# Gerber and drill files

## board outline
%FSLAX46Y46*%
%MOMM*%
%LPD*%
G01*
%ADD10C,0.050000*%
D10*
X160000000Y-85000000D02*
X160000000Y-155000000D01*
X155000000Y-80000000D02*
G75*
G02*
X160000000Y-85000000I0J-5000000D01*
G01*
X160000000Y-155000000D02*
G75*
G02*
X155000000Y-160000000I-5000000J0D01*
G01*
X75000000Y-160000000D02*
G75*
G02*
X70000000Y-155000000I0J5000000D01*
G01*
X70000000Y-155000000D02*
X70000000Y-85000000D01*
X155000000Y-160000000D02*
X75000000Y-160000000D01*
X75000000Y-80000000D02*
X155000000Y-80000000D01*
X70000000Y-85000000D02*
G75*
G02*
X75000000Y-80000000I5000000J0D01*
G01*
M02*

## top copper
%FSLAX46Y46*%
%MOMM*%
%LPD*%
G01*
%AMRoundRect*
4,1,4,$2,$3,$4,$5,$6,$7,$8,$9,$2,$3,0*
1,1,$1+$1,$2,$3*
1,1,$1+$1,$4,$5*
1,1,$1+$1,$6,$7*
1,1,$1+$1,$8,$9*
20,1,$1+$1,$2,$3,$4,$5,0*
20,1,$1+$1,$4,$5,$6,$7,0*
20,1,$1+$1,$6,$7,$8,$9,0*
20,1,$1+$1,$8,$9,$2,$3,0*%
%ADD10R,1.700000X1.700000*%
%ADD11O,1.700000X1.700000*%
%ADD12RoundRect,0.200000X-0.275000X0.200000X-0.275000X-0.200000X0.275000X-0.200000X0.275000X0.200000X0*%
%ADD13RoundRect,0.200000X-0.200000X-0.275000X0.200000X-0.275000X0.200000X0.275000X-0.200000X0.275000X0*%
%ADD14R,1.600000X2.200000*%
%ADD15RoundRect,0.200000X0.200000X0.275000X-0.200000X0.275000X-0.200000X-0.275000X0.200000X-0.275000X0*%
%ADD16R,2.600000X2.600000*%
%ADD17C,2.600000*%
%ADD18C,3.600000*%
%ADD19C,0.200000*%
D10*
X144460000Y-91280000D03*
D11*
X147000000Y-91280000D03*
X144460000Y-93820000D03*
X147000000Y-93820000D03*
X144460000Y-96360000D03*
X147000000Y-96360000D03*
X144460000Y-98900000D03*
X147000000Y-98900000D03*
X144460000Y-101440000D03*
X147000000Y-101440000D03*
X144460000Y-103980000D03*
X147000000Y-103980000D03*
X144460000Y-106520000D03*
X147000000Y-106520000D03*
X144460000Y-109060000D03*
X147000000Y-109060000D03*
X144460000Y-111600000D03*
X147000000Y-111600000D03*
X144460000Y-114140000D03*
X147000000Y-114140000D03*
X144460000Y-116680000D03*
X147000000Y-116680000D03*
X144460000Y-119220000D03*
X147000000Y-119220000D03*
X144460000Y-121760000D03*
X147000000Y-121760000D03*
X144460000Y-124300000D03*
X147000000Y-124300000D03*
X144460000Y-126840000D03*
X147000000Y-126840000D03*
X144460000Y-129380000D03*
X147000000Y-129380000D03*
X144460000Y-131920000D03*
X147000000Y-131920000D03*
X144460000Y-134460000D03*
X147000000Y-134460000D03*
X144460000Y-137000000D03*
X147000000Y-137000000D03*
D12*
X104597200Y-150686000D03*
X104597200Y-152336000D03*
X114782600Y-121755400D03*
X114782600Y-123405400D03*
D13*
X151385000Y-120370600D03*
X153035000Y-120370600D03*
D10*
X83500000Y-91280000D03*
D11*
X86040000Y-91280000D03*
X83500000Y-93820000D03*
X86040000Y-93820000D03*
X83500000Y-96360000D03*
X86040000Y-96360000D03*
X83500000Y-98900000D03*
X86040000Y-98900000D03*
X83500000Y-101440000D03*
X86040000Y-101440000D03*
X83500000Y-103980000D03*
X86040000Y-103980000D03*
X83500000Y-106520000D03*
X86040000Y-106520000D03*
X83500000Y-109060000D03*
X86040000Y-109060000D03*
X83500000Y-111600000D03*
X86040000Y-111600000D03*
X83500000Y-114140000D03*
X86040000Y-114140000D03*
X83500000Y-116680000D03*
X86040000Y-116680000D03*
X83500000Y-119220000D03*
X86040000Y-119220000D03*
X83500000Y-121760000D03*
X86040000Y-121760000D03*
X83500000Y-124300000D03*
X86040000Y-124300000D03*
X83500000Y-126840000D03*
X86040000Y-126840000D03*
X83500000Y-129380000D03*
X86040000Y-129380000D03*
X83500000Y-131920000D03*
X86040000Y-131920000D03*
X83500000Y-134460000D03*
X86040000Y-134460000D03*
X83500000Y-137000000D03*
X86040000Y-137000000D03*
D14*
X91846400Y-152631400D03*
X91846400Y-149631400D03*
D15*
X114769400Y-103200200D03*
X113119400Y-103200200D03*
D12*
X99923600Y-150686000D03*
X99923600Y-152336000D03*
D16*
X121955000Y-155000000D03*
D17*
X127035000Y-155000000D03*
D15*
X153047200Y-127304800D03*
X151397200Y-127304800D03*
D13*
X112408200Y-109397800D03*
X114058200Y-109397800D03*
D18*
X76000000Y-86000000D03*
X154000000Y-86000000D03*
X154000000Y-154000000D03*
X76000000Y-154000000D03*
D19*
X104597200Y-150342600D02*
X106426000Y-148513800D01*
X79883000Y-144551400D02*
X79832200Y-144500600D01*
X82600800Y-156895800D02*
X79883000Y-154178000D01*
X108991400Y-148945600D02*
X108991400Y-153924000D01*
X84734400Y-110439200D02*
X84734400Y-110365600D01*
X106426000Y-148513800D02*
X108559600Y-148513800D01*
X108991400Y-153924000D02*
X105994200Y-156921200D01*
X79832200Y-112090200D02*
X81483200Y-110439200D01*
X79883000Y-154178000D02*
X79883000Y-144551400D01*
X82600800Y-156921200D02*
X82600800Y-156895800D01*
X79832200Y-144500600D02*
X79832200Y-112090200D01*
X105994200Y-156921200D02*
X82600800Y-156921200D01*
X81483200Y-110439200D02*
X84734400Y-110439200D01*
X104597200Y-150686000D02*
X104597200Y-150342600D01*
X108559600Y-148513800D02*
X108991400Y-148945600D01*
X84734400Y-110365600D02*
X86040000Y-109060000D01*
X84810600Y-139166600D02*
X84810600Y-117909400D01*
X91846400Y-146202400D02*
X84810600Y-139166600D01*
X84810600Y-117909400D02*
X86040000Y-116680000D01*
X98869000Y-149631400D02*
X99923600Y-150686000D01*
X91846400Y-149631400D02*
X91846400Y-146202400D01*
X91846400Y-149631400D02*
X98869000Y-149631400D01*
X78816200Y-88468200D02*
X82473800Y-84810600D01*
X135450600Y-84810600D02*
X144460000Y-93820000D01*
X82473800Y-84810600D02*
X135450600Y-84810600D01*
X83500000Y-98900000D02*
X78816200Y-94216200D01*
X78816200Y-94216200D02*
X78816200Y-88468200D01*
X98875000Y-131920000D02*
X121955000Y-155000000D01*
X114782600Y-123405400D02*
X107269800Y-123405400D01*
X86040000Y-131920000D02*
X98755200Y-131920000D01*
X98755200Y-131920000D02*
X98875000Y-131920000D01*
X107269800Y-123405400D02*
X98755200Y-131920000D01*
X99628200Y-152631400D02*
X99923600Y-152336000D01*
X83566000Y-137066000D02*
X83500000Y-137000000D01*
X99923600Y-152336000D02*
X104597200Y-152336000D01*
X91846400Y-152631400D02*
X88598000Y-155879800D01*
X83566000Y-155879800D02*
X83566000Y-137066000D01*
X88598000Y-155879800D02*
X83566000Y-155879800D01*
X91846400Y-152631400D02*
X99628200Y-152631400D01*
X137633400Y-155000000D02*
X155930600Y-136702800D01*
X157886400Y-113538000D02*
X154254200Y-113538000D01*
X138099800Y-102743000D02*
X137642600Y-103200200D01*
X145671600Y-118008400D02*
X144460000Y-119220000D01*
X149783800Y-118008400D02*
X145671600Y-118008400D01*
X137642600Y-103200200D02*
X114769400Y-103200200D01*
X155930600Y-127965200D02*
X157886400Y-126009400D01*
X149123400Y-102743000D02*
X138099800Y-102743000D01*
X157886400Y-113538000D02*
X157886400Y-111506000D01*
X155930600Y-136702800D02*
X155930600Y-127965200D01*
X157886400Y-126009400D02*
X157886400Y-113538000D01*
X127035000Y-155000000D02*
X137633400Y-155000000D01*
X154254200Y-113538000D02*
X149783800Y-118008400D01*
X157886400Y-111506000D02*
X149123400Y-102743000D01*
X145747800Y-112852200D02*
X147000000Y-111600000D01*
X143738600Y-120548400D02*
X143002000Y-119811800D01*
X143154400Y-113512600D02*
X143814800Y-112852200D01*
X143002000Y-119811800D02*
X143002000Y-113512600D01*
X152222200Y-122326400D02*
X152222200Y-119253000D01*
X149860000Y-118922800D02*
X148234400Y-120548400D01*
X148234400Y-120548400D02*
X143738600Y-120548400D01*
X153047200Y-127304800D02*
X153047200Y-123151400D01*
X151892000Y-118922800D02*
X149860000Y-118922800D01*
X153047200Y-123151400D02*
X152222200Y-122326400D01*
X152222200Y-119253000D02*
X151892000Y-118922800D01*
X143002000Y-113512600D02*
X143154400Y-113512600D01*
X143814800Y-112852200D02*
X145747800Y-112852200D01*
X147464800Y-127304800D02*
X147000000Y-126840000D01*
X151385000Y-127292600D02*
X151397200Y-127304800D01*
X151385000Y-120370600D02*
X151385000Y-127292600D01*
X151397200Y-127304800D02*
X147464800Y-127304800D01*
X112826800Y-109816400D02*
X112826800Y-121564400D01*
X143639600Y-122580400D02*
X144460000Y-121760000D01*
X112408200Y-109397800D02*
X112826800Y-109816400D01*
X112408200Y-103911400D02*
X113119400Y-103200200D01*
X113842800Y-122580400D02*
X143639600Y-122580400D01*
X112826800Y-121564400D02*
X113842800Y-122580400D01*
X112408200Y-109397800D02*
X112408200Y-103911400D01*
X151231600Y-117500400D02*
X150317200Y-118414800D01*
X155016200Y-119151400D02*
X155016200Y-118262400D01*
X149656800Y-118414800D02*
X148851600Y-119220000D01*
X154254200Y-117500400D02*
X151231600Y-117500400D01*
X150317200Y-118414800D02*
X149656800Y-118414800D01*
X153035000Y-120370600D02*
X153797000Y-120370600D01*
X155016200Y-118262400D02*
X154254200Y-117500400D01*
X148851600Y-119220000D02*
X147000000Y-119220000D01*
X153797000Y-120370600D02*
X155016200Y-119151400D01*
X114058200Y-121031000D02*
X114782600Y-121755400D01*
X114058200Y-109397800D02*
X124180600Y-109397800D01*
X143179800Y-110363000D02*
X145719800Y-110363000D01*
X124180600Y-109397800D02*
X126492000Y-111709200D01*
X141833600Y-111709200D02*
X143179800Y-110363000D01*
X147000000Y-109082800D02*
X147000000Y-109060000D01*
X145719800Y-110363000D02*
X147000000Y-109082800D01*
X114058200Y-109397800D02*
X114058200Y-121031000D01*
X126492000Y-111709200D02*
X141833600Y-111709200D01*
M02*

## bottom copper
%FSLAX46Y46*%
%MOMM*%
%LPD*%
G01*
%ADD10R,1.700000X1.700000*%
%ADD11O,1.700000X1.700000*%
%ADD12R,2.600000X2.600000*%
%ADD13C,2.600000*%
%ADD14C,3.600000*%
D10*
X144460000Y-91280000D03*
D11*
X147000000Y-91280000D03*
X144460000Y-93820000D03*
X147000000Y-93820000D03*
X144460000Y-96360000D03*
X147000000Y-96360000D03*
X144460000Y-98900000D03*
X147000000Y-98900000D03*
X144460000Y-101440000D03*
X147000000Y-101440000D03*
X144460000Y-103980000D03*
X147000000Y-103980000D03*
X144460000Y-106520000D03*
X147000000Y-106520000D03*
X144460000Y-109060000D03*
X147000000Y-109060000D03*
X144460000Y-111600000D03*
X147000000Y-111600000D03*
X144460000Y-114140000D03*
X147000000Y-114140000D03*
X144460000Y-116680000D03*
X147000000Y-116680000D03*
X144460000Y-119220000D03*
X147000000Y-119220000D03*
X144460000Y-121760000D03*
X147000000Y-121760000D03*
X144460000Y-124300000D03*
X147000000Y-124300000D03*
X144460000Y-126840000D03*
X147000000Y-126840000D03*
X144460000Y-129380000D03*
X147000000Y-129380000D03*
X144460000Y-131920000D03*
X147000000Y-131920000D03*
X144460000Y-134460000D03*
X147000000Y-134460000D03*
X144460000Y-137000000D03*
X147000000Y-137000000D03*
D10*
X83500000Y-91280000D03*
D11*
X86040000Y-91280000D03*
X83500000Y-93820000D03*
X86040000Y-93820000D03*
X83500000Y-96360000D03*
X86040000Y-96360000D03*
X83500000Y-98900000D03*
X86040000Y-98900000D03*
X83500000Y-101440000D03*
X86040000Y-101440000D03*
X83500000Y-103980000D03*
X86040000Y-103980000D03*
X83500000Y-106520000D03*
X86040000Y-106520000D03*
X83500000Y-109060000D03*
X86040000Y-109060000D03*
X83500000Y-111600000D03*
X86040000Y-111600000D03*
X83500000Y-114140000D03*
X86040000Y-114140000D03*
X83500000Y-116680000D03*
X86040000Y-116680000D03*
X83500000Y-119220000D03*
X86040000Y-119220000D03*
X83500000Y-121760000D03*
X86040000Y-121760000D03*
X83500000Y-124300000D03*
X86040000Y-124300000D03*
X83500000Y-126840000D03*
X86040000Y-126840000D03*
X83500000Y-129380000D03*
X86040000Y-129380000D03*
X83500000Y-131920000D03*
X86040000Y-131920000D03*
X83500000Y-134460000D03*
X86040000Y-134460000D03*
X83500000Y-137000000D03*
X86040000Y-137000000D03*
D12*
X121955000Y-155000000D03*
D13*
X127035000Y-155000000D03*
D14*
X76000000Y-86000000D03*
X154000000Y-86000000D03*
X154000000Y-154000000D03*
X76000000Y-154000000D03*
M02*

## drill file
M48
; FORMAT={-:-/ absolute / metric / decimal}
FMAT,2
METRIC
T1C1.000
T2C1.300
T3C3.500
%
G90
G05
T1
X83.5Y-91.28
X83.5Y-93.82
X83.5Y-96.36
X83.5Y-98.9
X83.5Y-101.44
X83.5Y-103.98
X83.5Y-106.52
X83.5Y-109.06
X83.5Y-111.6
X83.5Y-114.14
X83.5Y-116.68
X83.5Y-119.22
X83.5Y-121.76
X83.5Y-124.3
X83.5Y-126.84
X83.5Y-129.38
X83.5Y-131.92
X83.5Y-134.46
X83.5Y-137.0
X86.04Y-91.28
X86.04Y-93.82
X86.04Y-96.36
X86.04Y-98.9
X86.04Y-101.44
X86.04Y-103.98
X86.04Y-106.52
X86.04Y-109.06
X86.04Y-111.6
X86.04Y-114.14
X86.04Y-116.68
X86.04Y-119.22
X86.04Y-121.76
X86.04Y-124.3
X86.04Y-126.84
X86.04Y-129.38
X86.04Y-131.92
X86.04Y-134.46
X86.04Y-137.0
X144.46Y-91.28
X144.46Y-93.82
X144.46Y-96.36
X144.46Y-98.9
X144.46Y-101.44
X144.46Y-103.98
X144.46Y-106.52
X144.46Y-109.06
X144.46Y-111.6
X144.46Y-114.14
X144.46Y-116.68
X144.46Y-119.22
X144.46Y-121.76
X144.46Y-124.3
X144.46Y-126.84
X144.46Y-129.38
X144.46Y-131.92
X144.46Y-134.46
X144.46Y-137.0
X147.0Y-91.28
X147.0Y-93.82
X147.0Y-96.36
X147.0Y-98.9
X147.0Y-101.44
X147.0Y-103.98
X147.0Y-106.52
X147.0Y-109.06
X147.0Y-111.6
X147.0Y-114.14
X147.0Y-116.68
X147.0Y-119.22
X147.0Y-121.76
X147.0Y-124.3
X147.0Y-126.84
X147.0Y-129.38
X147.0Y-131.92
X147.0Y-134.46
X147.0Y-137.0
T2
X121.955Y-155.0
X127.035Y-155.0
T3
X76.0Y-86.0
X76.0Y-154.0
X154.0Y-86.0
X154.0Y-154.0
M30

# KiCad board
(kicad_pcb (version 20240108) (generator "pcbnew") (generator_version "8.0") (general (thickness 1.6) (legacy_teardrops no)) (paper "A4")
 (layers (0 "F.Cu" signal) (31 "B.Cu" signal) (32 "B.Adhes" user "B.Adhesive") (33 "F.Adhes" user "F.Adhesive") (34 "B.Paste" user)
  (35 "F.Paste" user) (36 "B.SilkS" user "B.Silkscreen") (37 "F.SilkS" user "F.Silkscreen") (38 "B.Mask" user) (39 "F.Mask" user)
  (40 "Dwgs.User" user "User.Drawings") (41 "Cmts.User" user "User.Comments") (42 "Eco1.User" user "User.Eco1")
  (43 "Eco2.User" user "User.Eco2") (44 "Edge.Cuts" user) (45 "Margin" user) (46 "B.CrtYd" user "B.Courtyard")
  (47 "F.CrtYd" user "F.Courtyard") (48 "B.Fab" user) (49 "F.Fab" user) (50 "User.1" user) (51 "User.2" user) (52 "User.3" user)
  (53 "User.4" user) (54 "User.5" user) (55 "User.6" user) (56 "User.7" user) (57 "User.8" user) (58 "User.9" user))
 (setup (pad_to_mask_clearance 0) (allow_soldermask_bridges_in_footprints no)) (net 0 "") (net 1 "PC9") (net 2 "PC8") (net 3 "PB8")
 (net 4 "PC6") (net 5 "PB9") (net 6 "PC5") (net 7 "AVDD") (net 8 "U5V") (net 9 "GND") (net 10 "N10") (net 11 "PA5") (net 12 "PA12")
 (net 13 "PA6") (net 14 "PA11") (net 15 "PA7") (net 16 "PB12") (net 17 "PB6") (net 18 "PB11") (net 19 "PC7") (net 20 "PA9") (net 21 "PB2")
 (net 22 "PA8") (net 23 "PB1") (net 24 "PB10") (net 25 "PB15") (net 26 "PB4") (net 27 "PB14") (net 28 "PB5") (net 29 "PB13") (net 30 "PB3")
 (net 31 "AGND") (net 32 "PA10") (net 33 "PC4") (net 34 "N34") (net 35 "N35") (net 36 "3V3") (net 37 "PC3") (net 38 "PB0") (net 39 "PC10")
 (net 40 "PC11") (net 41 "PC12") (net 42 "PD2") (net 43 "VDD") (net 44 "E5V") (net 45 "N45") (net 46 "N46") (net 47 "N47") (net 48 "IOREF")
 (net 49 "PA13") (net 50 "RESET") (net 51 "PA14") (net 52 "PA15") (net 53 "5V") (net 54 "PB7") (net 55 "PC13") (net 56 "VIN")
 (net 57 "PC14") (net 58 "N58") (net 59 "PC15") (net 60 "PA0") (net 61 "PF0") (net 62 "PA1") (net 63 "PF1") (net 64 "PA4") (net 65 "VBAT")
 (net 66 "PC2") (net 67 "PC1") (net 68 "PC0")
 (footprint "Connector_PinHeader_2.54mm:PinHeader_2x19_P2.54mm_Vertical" (layer "F.Cu") (at 144.46 91.28)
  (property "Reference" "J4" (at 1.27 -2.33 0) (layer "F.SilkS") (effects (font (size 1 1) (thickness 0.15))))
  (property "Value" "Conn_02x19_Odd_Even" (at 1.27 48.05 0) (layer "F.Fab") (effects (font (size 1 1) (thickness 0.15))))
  (pad "1" thru_hole rect (at 0 0) (size 1.7 1.7) (drill 1) (layers "*.Cu" "*.Mask") (remove_unused_layers no) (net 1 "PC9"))
  (pad "2" thru_hole oval (at 2.54 0) (size 1.7 1.7) (drill 1) (layers "*.Cu" "*.Mask") (remove_unused_layers no) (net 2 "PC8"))
  (pad "3" thru_hole oval (at 0 2.54) (size 1.7 1.7) (drill 1) (layers "*.Cu" "*.Mask") (remove_unused_layers no) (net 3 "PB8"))
  (pad "4" thru_hole oval (at 2.54 2.54) (size 1.7 1.7) (drill 1) (layers "*.Cu" "*.Mask") (remove_unused_layers no) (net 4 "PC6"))
  (pad "5" thru_hole oval (at 0 5.08) (size 1.7 1.7) (drill 1) (layers "*.Cu" "*.Mask") (remove_unused_layers no) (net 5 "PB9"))
  (pad "6" thru_hole oval (at 2.54 5.08) (size 1.7 1.7) (drill 1) (layers "*.Cu" "*.Mask") (remove_unused_layers no) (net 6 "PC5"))
  (pad "7" thru_hole oval (at 0 7.62) (size 1.7 1.7) (drill 1) (layers "*.Cu" "*.Mask") (remove_unused_layers no) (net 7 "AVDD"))
  (pad "8" thru_hole oval (at 2.54 7.62) (size 1.7 1.7) (drill 1) (layers "*.Cu" "*.Mask") (remove_unused_layers no) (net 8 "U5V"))
  (pad "9" thru_hole oval (at 0 10.16) (size 1.7 1.7) (drill 1) (layers "*.Cu" "*.Mask") (remove_unused_layers no) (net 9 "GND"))
  (pad "10" thru_hole oval (at 2.54 10.16) (size 1.7 1.7) (drill 1) (layers "*.Cu" "*.Mask") (remove_unused_layers no) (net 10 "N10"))
  (pad "11" thru_hole oval (at 0 12.7) (size 1.7 1.7) (drill 1) (layers "*.Cu" "*.Mask") (remove_unused_layers no) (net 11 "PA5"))
  (pad "12" thru_hole oval (at 2.54 12.7) (size 1.7 1.7) (drill 1) (layers "*.Cu" "*.Mask") (remove_unused_layers no) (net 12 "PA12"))
  (pad "13" thru_hole oval (at 0 15.24) (size 1.7 1.7) (drill 1) (layers "*.Cu" "*.Mask") (remove_unused_layers no) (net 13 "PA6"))
  (pad "14" thru_hole oval (at 2.54 15.24) (size 1.7 1.7) (drill 1) (layers "*.Cu" "*.Mask") (remove_unused_layers no) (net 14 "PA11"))
  (pad "15" thru_hole oval (at 0 17.78) (size 1.7 1.7) (drill 1) (layers "*.Cu" "*.Mask") (remove_unused_layers no) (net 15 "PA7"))
  (pad "16" thru_hole oval (at 2.54 17.78) (size 1.7 1.7) (drill 1) (layers "*.Cu" "*.Mask") (remove_unused_layers no) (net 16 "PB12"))
  (pad "17" thru_hole oval (at 0 20.32) (size 1.7 1.7) (drill 1) (layers "*.Cu" "*.Mask") (remove_unused_layers no) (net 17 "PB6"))
  (pad "18" thru_hole oval (at 2.54 20.32) (size 1.7 1.7) (drill 1) (layers "*.Cu" "*.Mask") (remove_unused_layers no) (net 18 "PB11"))
  (pad "19" thru_hole oval (at 0 22.86) (size 1.7 1.7) (drill 1) (layers "*.Cu" "*.Mask") (remove_unused_layers no) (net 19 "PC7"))
  (pad "20" thru_hole oval (at 2.54 22.86) (size 1.7 1.7) (drill 1) (layers "*.Cu" "*.Mask") (remove_unused_layers no) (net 9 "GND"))
  (pad "21" thru_hole oval (at 0 25.4) (size 1.7 1.7) (drill 1) (layers "*.Cu" "*.Mask") (remove_unused_layers no) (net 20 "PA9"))
  (pad "22" thru_hole oval (at 2.54 25.4) (size 1.7 1.7) (drill 1) (layers "*.Cu" "*.Mask") (remove_unused_layers no) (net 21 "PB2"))
  (pad "23" thru_hole oval (at 0 27.94) (size 1.7 1.7) (drill 1) (layers "*.Cu" "*.Mask") (remove_unused_layers no) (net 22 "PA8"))
  (pad "24" thru_hole oval (at 2.54 27.94) (size 1.7 1.7) (drill 1) (layers "*.Cu" "*.Mask") (remove_unused_layers no) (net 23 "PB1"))
  (pad "25" thru_hole oval (at 0 30.48) (size 1.7 1.7) (drill 1) (layers "*.Cu" "*.Mask") (remove_unused_layers no) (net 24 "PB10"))
  (pad "26" thru_hole oval (at 2.54 30.48) (size 1.7 1.7) (drill 1) (layers "*.Cu" "*.Mask") (remove_unused_layers no) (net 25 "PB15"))
  (pad "27" thru_hole oval (at 0 33.02) (size 1.7 1.7) (drill 1) (layers "*.Cu" "*.Mask") (remove_unused_layers no) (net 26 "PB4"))
  (pad "28" thru_hole oval (at 2.54 33.02) (size 1.7 1.7) (drill 1) (layers "*.Cu" "*.Mask") (remove_unused_layers no) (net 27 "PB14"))
  (pad "29" thru_hole oval (at 0 35.56) (size 1.7 1.7) (drill 1) (layers "*.Cu" "*.Mask") (remove_unused_layers no) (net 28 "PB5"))
  (pad "30" thru_hole oval (at 2.54 35.56) (size 1.7 1.7) (drill 1) (layers "*.Cu" "*.Mask") (remove_unused_layers no) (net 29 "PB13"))
  (pad "31" thru_hole oval (at 0 38.1) (size 1.7 1.7) (drill 1) (layers "*.Cu" "*.Mask") (remove_unused_layers no) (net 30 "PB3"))
  (pad "32" thru_hole oval (at 2.54 38.1) (size 1.7 1.7) (drill 1) (layers "*.Cu" "*.Mask") (remove_unused_layers no) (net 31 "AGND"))
  (pad "33" thru_hole oval (at 0 40.64) (size 1.7 1.7) (drill 1) (layers "*.Cu" "*.Mask") (remove_unused_layers no) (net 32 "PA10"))
  (pad "34" thru_hole oval (at 2.54 40.64) (size 1.7 1.7) (drill 1) (layers "*.Cu" "*.Mask") (remove_unused_layers no) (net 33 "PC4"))
  (pad "35" thru_hole oval (at 0 43.18) (size 1.7 1.7) (drill 1) (layers "*.Cu" "*.Mask") (remove_unused_layers no) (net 33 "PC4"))
  (pad "36" thru_hole oval (at 2.54 43.18) (size 1.7 1.7) (drill 1) (layers "*.Cu" "*.Mask") (remove_unused_layers no) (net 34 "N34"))
  (pad "37" thru_hole oval (at 0 45.72) (size 1.7 1.7) (drill 1) (layers "*.Cu" "*.Mask") (remove_unused_layers no) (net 6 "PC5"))
  (pad "38" thru_hole oval (at 2.54 45.72) (size 1.7 1.7) (drill 1) (layers "*.Cu" "*.Mask") (remove_unused_layers no) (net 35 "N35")))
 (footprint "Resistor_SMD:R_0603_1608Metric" (layer "F.Cu") (at 104.5972 151.511 -90)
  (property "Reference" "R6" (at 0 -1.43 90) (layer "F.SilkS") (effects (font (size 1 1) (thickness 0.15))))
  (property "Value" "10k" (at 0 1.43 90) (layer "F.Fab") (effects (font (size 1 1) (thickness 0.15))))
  (pad "1" smd roundrect (at -0.825 0 270) (size 0.8 0.95) (layers "F.Cu" "F.Paste" "F.Mask") (roundrect_rratio 0.25) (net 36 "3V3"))
  (pad "2" smd roundrect (at 0.825 0 270) (size 0.8 0.95) (layers "F.Cu" "F.Paste" "F.Mask") (roundrect_rratio 0.25) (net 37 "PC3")))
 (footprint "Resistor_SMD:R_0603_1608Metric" (layer "F.Cu") (at 114.7826 122.5804 -90)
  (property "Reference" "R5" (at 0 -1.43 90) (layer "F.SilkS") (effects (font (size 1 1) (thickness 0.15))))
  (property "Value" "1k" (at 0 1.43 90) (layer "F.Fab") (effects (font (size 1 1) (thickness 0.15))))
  (pad "1" smd roundrect (at -0.825 0 270) (size 0.8 0.95) (layers "F.Cu" "F.Paste" "F.Mask") (roundrect_rratio 0.25) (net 16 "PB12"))
  (pad "2" smd roundrect (at 0.825 0 270) (size 0.8 0.95) (layers "F.Cu" "F.Paste" "F.Mask") (roundrect_rratio 0.25) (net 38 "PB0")))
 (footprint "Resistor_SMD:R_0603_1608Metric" (layer "F.Cu") (at 152.21 120.3706)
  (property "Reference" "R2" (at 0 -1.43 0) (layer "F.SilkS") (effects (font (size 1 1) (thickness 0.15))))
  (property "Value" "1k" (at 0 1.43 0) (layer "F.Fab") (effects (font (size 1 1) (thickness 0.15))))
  (pad "1" smd roundrect (at -0.825 0) (size 0.8 0.95) (layers "F.Cu" "F.Paste" "F.Mask") (roundrect_rratio 0.25) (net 29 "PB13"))
  (pad "2" smd roundrect (at 0.825 0) (size 0.8 0.95) (layers "F.Cu" "F.Paste" "F.Mask") (roundrect_rratio 0.25) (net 23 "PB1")))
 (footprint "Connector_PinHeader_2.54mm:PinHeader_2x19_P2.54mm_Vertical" (layer "F.Cu") (at 83.5 91.28)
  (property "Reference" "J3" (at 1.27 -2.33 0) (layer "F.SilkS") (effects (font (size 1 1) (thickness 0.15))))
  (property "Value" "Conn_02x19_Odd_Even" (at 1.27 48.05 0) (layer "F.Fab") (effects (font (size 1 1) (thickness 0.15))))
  (pad "1" thru_hole rect (at 0 0) (size 1.7 1.7) (drill 1) (layers "*.Cu" "*.Mask") (remove_unused_layers no) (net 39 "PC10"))
  (pad "2" thru_hole oval (at 2.54 0) (size 1.7 1.7) (drill 1) (layers "*.Cu" "*.Mask") (remove_unused_layers no) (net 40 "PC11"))
  (pad "3" thru_hole oval (at 0 2.54) (size 1.7 1.7) (drill 1) (layers "*.Cu" "*.Mask") (remove_unused_layers no) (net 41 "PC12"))
  (pad "4" thru_hole oval (at 2.54 2.54) (size 1.7 1.7) (drill 1) (layers "*.Cu" "*.Mask") (remove_unused_layers no) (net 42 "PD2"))
  (pad "5" thru_hole oval (at 0 5.08) (size 1.7 1.7) (drill 1) (layers "*.Cu" "*.Mask") (remove_unused_layers no) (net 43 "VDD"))
  (pad "6" thru_hole oval (at 2.54 5.08) (size 1.7 1.7) (drill 1) (layers "*.Cu" "*.Mask") (remove_unused_layers no) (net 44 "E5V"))
  (pad "7" thru_hole oval (at 0 7.62) (size 1.7 1.7) (drill 1) (layers "*.Cu" "*.Mask") (remove_unused_layers no) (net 3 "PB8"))
  (pad "8" thru_hole oval (at 2.54 7.62) (size 1.7 1.7) (drill 1) (layers "*.Cu" "*.Mask") (remove_unused_layers no) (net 9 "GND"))
  (pad "9" thru_hole oval (at 0 10.16) (size 1.7 1.7) (drill 1) (layers "*.Cu" "*.Mask") (remove_unused_layers no) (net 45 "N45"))
  (pad "10" thru_hole oval (at 2.54 10.16) (size 1.7 1.7) (drill 1) (layers "*.Cu" "*.Mask") (remove_unused_layers no) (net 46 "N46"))
  (pad "11" thru_hole oval (at 0 12.7) (size 1.7 1.7) (drill 1) (layers "*.Cu" "*.Mask") (remove_unused_layers no) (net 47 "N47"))
  (pad "12" thru_hole oval (at 2.54 12.7) (size 1.7 1.7) (drill 1) (layers "*.Cu" "*.Mask") (remove_unused_layers no) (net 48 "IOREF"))
  (pad "13" thru_hole oval (at 0 15.24) (size 1.7 1.7) (drill 1) (layers "*.Cu" "*.Mask") (remove_unused_layers no) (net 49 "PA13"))
  (pad "14" thru_hole oval (at 2.54 15.24) (size 1.7 1.7) (drill 1) (layers "*.Cu" "*.Mask") (remove_unused_layers no) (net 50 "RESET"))
  (pad "15" thru_hole oval (at 0 17.78) (size 1.7 1.7) (drill 1) (layers "*.Cu" "*.Mask") (remove_unused_layers no) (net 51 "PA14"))
  (pad "16" thru_hole oval (at 2.54 17.78) (size 1.7 1.7) (drill 1) (layers "*.Cu" "*.Mask") (remove_unused_layers no) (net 36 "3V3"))
  (pad "17" thru_hole oval (at 0 20.32) (size 1.7 1.7) (drill 1) (layers "*.Cu" "*.Mask") (remove_unused_layers no) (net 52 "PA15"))
  (pad "18" thru_hole oval (at 2.54 20.32) (size 1.7 1.7) (drill 1) (layers "*.Cu" "*.Mask") (remove_unused_layers no) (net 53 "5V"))
  (pad "19" thru_hole oval (at 0 22.86) (size 1.7 1.7) (drill 1) (layers "*.Cu" "*.Mask") (remove_unused_layers no) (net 9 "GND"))
  (pad "20" thru_hole oval (at 2.54 22.86) (size 1.7 1.7) (drill 1) (layers "*.Cu" "*.Mask") (remove_unused_layers no) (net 9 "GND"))
  (pad "21" thru_hole oval (at 0 25.4) (size 1.7 1.7) (drill 1) (layers "*.Cu" "*.Mask") (remove_unused_layers no) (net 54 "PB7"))
  (pad "22" thru_hole oval (at 2.54 25.4) (size 1.7 1.7) (drill 1) (layers "*.Cu" "*.Mask") (remove_unused_layers no) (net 9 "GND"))
  (pad "23" thru_hole oval (at 0 27.94) (size 1.7 1.7) (drill 1) (layers "*.Cu" "*.Mask") (remove_unused_layers no) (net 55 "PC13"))
  (pad "24" thru_hole oval (at 2.54 27.94) (size 1.7 1.7) (drill 1) (layers "*.Cu" "*.Mask") (remove_unused_layers no) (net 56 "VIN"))
  (pad "25" thru_hole oval (at 0 30.48) (size 1.7 1.7) (drill 1) (layers "*.Cu" "*.Mask") (remove_unused_layers no) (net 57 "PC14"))
  (pad "26" thru_hole oval (at 2.54 30.48) (size 1.7 1.7) (drill 1) (layers "*.Cu" "*.Mask") (remove_unused_layers no) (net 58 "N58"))
  (pad "27" thru_hole oval (at 0 33.02) (size 1.7 1.7) (drill 1) (layers "*.Cu" "*.Mask") (remove_unused_layers no) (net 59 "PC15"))
  (pad "28" thru_hole oval (at 2.54 33.02) (size 1.7 1.7) (drill 1) (layers "*.Cu" "*.Mask") (remove_unused_layers no) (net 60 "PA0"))
  (pad "29" thru_hole oval (at 0 35.56) (size 1.7 1.7) (drill 1) (layers "*.Cu" "*.Mask") (remove_unused_layers no) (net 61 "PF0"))
  (pad "30" thru_hole oval (at 2.54 35.56) (size 1.7 1.7) (drill 1) (layers "*.Cu" "*.Mask") (remove_unused_layers no) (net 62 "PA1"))
  (pad "31" thru_hole oval (at 0 38.1) (size 1.7 1.7) (drill 1) (layers "*.Cu" "*.Mask") (remove_unused_layers no) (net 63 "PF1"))
  (pad "32" thru_hole oval (at 2.54 38.1) (size 1.7 1.7) (drill 1) (layers "*.Cu" "*.Mask") (remove_unused_layers no) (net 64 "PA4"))
  (pad "33" thru_hole oval (at 0 40.64) (size 1.7 1.7) (drill 1) (layers "*.Cu" "*.Mask") (remove_unused_layers no) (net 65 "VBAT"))
  (pad "34" thru_hole oval (at 2.54 40.64) (size 1.7 1.7) (drill 1) (layers "*.Cu" "*.Mask") (remove_unused_layers no) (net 38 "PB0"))
  (pad "35" thru_hole oval (at 0 43.18) (size 1.7 1.7) (drill 1) (layers "*.Cu" "*.Mask") (remove_unused_layers no) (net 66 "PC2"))
  (pad "36" thru_hole oval (at 2.54 43.18) (size 1.7 1.7) (drill 1) (layers "*.Cu" "*.Mask") (remove_unused_layers no) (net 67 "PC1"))
  (pad "37" thru_hole oval (at 0 45.72) (size 1.7 1.7) (drill 1) (layers "*.Cu" "*.Mask") (remove_unused_layers no) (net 37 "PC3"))
  (pad "38" thru_hole oval (at 2.54 45.72) (size 1.7 1.7) (drill 1) (layers "*.Cu" "*.Mask") (remove_unused_layers no) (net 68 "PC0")))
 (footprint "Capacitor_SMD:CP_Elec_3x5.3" (layer "F.Cu") (at 91.8464 151.1314 90)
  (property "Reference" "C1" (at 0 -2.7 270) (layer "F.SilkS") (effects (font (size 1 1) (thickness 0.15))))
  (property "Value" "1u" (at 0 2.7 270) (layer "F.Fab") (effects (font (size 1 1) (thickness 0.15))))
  (pad "1" smd rect (at -1.5 0 90) (size 2.2 1.6) (layers "F.Cu" "F.Paste" "F.Mask") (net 37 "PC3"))
  (pad "2" smd rect (at 1.5 0 90) (size 2.2 1.6) (layers "F.Cu" "F.Paste" "F.Mask") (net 9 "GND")))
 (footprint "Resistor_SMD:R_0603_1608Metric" (layer "F.Cu") (at 113.9444 103.2002 180)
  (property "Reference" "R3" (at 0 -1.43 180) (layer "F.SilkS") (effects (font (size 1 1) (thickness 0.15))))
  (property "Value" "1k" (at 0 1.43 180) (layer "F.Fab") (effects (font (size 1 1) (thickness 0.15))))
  (pad "1" smd roundrect (at -0.825 0 180) (size 0.8 0.95) (layers "F.Cu" "F.Paste" "F.Mask") (roundrect_rratio 0.25) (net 22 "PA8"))
  (pad "2" smd roundrect (at 0.825 0 180) (size 0.8 0.95) (layers "F.Cu" "F.Paste" "F.Mask") (roundrect_rratio 0.25) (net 24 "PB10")))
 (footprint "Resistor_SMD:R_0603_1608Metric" (layer "F.Cu") (at 99.9236 151.511 -90)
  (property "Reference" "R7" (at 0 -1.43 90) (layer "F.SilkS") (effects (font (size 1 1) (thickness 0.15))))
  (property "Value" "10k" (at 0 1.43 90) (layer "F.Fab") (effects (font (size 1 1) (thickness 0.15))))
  (pad "1" smd roundrect (at -0.825 0 270) (size 0.8 0.95) (layers "F.Cu" "F.Paste" "F.Mask") (roundrect_rratio 0.25) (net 9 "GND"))
  (pad "2" smd roundrect (at 0.825 0 270) (size 0.8 0.95) (layers "F.Cu" "F.Paste" "F.Mask") (roundrect_rratio 0.25) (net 37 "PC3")))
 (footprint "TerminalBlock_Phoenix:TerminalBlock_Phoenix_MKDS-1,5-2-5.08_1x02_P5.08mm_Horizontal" (layer "F.Cu") (at 121.955 155)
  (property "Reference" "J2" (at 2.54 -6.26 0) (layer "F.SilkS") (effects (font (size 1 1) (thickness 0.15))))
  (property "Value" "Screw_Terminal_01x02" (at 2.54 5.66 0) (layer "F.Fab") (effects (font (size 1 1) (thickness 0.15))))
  (pad "1" thru_hole rect (at 0 0) (size 2.6 2.6) (drill 1.3) (layers "*.Cu" "*.Mask") (remove_unused_layers no) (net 38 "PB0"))
  (pad "2" thru_hole circle (at 5.08 0) (size 2.6 2.6) (drill 1.3) (layers "*.Cu" "*.Mask") (remove_unused_layers no) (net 22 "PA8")))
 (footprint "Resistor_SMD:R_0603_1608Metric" (layer "F.Cu") (at 152.2222 127.3048 180)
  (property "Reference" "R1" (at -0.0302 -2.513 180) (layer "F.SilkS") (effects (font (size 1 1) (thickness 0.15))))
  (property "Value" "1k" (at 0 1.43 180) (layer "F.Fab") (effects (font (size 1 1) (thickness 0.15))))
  (pad "1" smd roundrect (at -0.825 0 180) (size 0.8 0.95) (layers "F.Cu" "F.Paste" "F.Mask") (roundrect_rratio 0.25) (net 18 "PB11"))
  (pad "2" smd roundrect (at 0.825 0 180) (size 0.8 0.95) (layers "F.Cu" "F.Paste" "F.Mask") (roundrect_rratio 0.25) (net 29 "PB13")))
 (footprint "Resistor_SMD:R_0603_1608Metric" (layer "F.Cu") (at 113.2332 109.3978)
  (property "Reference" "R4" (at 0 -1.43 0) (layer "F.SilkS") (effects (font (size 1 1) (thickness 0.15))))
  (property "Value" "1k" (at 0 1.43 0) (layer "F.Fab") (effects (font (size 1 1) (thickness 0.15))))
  (pad "1" smd roundrect (at -0.825 0) (size 0.8 0.95) (layers "F.Cu" "F.Paste" "F.Mask") (roundrect_rratio 0.25) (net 24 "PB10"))
  (pad "2" smd roundrect (at 0.825 0) (size 0.8 0.95) (layers "F.Cu" "F.Paste" "F.Mask") (roundrect_rratio 0.25) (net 16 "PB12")))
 (gr_line (start 160 85) (end 160 155) (stroke (width 0.05) (type default)) (layer "Edge.Cuts"))
 (gr_arc (start 155 80) (mid 158.535534 81.464466) (end 160 85) (stroke (width 0.05) (type default)) (layer "Edge.Cuts"))
 (gr_arc (start 160 155) (mid 158.535534 158.535534) (end 155 160) (stroke (width 0.05) (type default)) (layer "Edge.Cuts"))
 (gr_arc (start 75 160) (mid 71.464466 158.535534) (end 70 155) (stroke (width 0.05) (type default)) (layer "Edge.Cuts"))
 (gr_line (start 70 155) (end 70 85) (stroke (width 0.05) (type default)) (layer "Edge.Cuts"))
 (gr_line (start 155 160) (end 75 160) (stroke (width 0.05) (type default)) (layer "Edge.Cuts"))
 (gr_line (start 75 80) (end 155 80) (stroke (width 0.05) (type default)) (layer "Edge.Cuts"))
 (gr_arc (start 70 85) (mid 71.464466 81.464466) (end 75 80) (stroke (width 0.05) (type default)) (layer "Edge.Cuts"))
 (via (at 76 86) (size 3.6) (drill 3.5) (layers "F.Cu" "B.Cu") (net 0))
 (via (at 154 86) (size 3.6) (drill 3.5) (layers "F.Cu" "B.Cu") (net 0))
 (via (at 154 154) (size 3.6) (drill 3.5) (layers "F.Cu" "B.Cu") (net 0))
 (via (at 76 154) (size 3.6) (drill 3.5) (layers "F.Cu" "B.Cu") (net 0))
 (segment (start 104.5972 150.3426) (end 106.426 148.5138) (width 0.2) (layer "F.Cu") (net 36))
 (segment (start 79.883 144.5514) (end 79.8322 144.5006) (width 0.2) (layer "F.Cu") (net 36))
 (segment (start 82.6008 156.8958) (end 79.883 154.178) (width 0.2) (layer "F.Cu") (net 36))
 (segment (start 108.9914 148.9456) (end 108.9914 153.924) (width 0.2) (layer "F.Cu") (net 36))
 (segment (start 84.7344 110.4392) (end 84.7344 110.3656) (width 0.2) (layer "F.Cu") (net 36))
 (segment (start 106.426 148.5138) (end 108.5596 148.5138) (width 0.2) (layer "F.Cu") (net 36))
 (segment (start 108.9914 153.924) (end 105.9942 156.9212) (width 0.2) (layer "F.Cu") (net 36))
 (segment (start 79.8322 112.0902) (end 81.4832 110.4392) (width 0.2) (layer "F.Cu") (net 36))
 (segment (start 79.883 154.178) (end 79.883 144.5514) (width 0.2) (layer "F.Cu") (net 36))
 (segment (start 82.6008 156.9212) (end 82.6008 156.8958) (width 0.2) (layer "F.Cu") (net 36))
 (segment (start 79.8322 144.5006) (end 79.8322 112.0902) (width 0.2) (layer "F.Cu") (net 36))
 (segment (start 105.9942 156.9212) (end 82.6008 156.9212) (width 0.2) (layer "F.Cu") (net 36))
 (segment (start 81.4832 110.4392) (end 84.7344 110.4392) (width 0.2) (layer "F.Cu") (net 36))
 (segment (start 104.5972 150.686) (end 104.5972 150.3426) (width 0.2) (layer "F.Cu") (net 36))
 (segment (start 108.5596 148.5138) (end 108.9914 148.9456) (width 0.2) (layer "F.Cu") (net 36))
 (segment (start 84.7344 110.3656) (end 86.04 109.06) (width 0.2) (layer "F.Cu") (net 36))
 (segment (start 84.8106 139.1666) (end 84.8106 117.9094) (width 0.2) (layer "F.Cu") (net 9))
 (segment (start 91.8464 146.2024) (end 84.8106 139.1666) (width 0.2) (layer "F.Cu") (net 9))
 (segment (start 84.8106 117.9094) (end 86.04 116.68) (width 0.2) (layer "F.Cu") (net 9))
 (segment (start 98.869 149.6314) (end 99.9236 150.686) (width 0.2) (layer "F.Cu") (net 9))
 (segment (start 91.8464 149.6314) (end 91.8464 146.2024) (width 0.2) (layer "F.Cu") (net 9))
 (segment (start 91.8464 149.6314) (end 98.869 149.6314) (width 0.2) (layer "F.Cu") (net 9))
 (segment (start 78.8162 88.4682) (end 82.4738 84.8106) (width 0.2) (layer "F.Cu") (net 3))
 (segment (start 135.4506 84.8106) (end 144.46 93.82) (width 0.2) (layer "F.Cu") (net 3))
 (segment (start 82.4738 84.8106) (end 135.4506 84.8106) (width 0.2) (layer "F.Cu") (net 3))
 (segment (start 83.5 98.9) (end 78.8162 94.2162) (width 0.2) (layer "F.Cu") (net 3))
 (segment (start 78.8162 94.2162) (end 78.8162 88.4682) (width 0.2) (layer "F.Cu") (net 3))
 (segment (start 98.875 131.92) (end 121.955 155) (width 0.2) (layer "F.Cu") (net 38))
 (segment (start 114.7826 123.4054) (end 107.2698 123.4054) (width 0.2) (layer "F.Cu") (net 38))
 (segment (start 86.04 131.92) (end 98.7552 131.92) (width 0.2) (layer "F.Cu") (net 38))
 (segment (start 98.7552 131.92) (end 98.875 131.92) (width 0.2) (layer "F.Cu") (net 38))
 (segment (start 107.2698 123.4054) (end 98.7552 131.92) (width 0.2) (layer "F.Cu") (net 38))
 (segment (start 99.6282 152.6314) (end 99.9236 152.336) (width 0.2) (layer "F.Cu") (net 37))
 (segment (start 83.566 137.066) (end 83.5 137) (width 0.2) (layer "F.Cu") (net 37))
 (segment (start 99.9236 152.336) (end 104.5972 152.336) (width 0.2) (layer "F.Cu") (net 37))
 (segment (start 91.8464 152.6314) (end 88.598 155.8798) (width 0.2) (layer "F.Cu") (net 37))
 (segment (start 83.566 155.8798) (end 83.566 137.066) (width 0.2) (layer "F.Cu") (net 37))
 (segment (start 88.598 155.8798) (end 83.566 155.8798) (width 0.2) (layer "F.Cu") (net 37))
 (segment (start 91.8464 152.6314) (end 99.6282 152.6314) (width 0.2) (layer "F.Cu") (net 37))
 (segment (start 137.6334 155) (end 155.9306 136.7028) (width 0.2) (layer "F.Cu") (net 22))
 (segment (start 157.8864 113.538) (end 154.2542 113.538) (width 0.2) (layer "F.Cu") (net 22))
 (segment (start 138.0998 102.743) (end 137.6426 103.2002) (width 0.2) (layer "F.Cu") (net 22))
 (segment (start 145.6716 118.0084) (end 144.46 119.22) (width 0.2) (layer "F.Cu") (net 22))
 (segment (start 149.7838 118.0084) (end 145.6716 118.0084) (width 0.2) (layer "F.Cu") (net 22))
 (segment (start 137.6426 103.2002) (end 114.7694 103.2002) (width 0.2) (layer "F.Cu") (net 22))
 (segment (start 155.9306 127.9652) (end 157.8864 126.0094) (width 0.2) (layer "F.Cu") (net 22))
 (segment (start 149.1234 102.743) (end 138.0998 102.743) (width 0.2) (layer "F.Cu") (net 22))
 (segment (start 157.8864 113.538) (end 157.8864 111.506) (width 0.2) (layer "F.Cu") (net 22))
 (segment (start 155.9306 136.7028) (end 155.9306 127.9652) (width 0.2) (layer "F.Cu") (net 22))
 (segment (start 157.8864 126.0094) (end 157.8864 113.538) (width 0.2) (layer "F.Cu") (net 22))
 (segment (start 127.035 155) (end 137.6334 155) (width 0.2) (layer "F.Cu") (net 22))
 (segment (start 154.2542 113.538) (end 149.7838 118.0084) (width 0.2) (layer "F.Cu") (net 22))
 (segment (start 157.8864 111.506) (end 149.1234 102.743) (width 0.2) (layer "F.Cu") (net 22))
 (segment (start 145.7478 112.8522) (end 147 111.6) (width 0.2) (layer "F.Cu") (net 18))
 (segment (start 143.7386 120.5484) (end 143.002 119.8118) (width 0.2) (layer "F.Cu") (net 18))
 (segment (start 143.1544 113.5126) (end 143.8148 112.8522) (width 0.2) (layer "F.Cu") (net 18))
 (segment (start 143.002 119.8118) (end 143.002 113.5126) (width 0.2) (layer "F.Cu") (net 18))
 (segment (start 152.2222 122.3264) (end 152.2222 119.253) (width 0.2) (layer "F.Cu") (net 18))
 (segment (start 149.86 118.9228) (end 148.2344 120.5484) (width 0.2) (layer "F.Cu") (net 18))
 (segment (start 148.2344 120.5484) (end 143.7386 120.5484) (width 0.2) (layer "F.Cu") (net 18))
 (segment (start 153.0472 127.3048) (end 153.0472 123.1514) (width 0.2) (layer "F.Cu") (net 18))
 (segment (start 151.892 118.9228) (end 149.86 118.9228) (width 0.2) (layer "F.Cu") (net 18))
 (segment (start 153.0472 123.1514) (end 152.2222 122.3264) (width 0.2) (layer "F.Cu") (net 18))
 (segment (start 152.2222 119.253) (end 151.892 118.9228) (width 0.2) (layer "F.Cu") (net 18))
 (segment (start 143.002 113.5126) (end 143.1544 113.5126) (width 0.2) (layer "F.Cu") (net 18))
 (segment (start 143.8148 112.8522) (end 145.7478 112.8522) (width 0.2) (layer "F.Cu") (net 18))
 (segment (start 147.4648 127.3048) (end 147 126.84) (width 0.2) (layer "F.Cu") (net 29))
 (segment (start 151.385 127.2926) (end 151.3972 127.3048) (width 0.2) (layer "F.Cu") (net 29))
 (segment (start 151.385 120.3706) (end 151.385 127.2926) (width 0.2) (layer "F.Cu") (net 29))
 (segment (start 151.3972 127.3048) (end 147.4648 127.3048) (width 0.2) (layer "F.Cu") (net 29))
 (segment (start 112.8268 109.8164) (end 112.8268 121.5644) (width 0.2) (layer "F.Cu") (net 24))
 (segment (start 143.6396 122.5804) (end 144.46 121.76) (width 0.2) (layer "F.Cu") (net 24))
 (segment (start 112.4082 109.3978) (end 112.8268 109.8164) (width 0.2) (layer "F.Cu") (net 24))
 (segment (start 112.4082 103.9114) (end 113.1194 103.2002) (width 0.2) (layer "F.Cu") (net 24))
 (segment (start 113.8428 122.5804) (end 143.6396 122.5804) (width 0.2) (layer "F.Cu") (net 24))
 (segment (start 112.8268 121.5644) (end 113.8428 122.5804) (width 0.2) (layer "F.Cu") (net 24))
 (segment (start 112.4082 109.3978) (end 112.4082 103.9114) (width 0.2) (layer "F.Cu") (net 24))
 (segment (start 151.2316 117.5004) (end 150.3172 118.4148) (width 0.2) (layer "F.Cu") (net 23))
 (segment (start 155.0162 119.1514) (end 155.0162 118.2624) (width 0.2) (layer "F.Cu") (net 23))
 (segment (start 149.6568 118.4148) (end 148.8516 119.22) (width 0.2) (layer "F.Cu") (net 23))
 (segment (start 154.2542 117.5004) (end 151.2316 117.5004) (width 0.2) (layer "F.Cu") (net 23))
 (segment (start 150.3172 118.4148) (end 149.6568 118.4148) (width 0.2) (layer "F.Cu") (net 23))
 (segment (start 153.035 120.3706) (end 153.797 120.3706) (width 0.2) (layer "F.Cu") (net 23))
 (segment (start 155.0162 118.2624) (end 154.2542 117.5004) (width 0.2) (layer "F.Cu") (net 23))
 (segment (start 148.8516 119.22) (end 147 119.22) (width 0.2) (layer "F.Cu") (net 23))
 (segment (start 153.797 120.3706) (end 155.0162 119.1514) (width 0.2) (layer "F.Cu") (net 23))
 (segment (start 114.0582 121.031) (end 114.7826 121.7554) (width 0.2) (layer "F.Cu") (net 16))
 (segment (start 114.0582 109.3978) (end 124.1806 109.3978) (width 0.2) (layer "F.Cu") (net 16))
 (segment (start 143.1798 110.363) (end 145.7198 110.363) (width 0.2) (layer "F.Cu") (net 16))
 (segment (start 124.1806 109.3978) (end 126.492 111.7092) (width 0.2) (layer "F.Cu") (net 16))
 (segment (start 141.8336 111.7092) (end 143.1798 110.363) (width 0.2) (layer "F.Cu") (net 16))
 (segment (start 147 109.0828) (end 147 109.06) (width 0.2) (layer "F.Cu") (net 16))
 (segment (start 145.7198 110.363) (end 147 109.0828) (width 0.2) (layer "F.Cu") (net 16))
 (segment (start 114.0582 109.3978) (end 114.0582 121.031) (width 0.2) (layer "F.Cu") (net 16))
 (segment (start 126.492 111.7092) (end 141.8336 111.7092) (width 0.2) (layer "F.Cu") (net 16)))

